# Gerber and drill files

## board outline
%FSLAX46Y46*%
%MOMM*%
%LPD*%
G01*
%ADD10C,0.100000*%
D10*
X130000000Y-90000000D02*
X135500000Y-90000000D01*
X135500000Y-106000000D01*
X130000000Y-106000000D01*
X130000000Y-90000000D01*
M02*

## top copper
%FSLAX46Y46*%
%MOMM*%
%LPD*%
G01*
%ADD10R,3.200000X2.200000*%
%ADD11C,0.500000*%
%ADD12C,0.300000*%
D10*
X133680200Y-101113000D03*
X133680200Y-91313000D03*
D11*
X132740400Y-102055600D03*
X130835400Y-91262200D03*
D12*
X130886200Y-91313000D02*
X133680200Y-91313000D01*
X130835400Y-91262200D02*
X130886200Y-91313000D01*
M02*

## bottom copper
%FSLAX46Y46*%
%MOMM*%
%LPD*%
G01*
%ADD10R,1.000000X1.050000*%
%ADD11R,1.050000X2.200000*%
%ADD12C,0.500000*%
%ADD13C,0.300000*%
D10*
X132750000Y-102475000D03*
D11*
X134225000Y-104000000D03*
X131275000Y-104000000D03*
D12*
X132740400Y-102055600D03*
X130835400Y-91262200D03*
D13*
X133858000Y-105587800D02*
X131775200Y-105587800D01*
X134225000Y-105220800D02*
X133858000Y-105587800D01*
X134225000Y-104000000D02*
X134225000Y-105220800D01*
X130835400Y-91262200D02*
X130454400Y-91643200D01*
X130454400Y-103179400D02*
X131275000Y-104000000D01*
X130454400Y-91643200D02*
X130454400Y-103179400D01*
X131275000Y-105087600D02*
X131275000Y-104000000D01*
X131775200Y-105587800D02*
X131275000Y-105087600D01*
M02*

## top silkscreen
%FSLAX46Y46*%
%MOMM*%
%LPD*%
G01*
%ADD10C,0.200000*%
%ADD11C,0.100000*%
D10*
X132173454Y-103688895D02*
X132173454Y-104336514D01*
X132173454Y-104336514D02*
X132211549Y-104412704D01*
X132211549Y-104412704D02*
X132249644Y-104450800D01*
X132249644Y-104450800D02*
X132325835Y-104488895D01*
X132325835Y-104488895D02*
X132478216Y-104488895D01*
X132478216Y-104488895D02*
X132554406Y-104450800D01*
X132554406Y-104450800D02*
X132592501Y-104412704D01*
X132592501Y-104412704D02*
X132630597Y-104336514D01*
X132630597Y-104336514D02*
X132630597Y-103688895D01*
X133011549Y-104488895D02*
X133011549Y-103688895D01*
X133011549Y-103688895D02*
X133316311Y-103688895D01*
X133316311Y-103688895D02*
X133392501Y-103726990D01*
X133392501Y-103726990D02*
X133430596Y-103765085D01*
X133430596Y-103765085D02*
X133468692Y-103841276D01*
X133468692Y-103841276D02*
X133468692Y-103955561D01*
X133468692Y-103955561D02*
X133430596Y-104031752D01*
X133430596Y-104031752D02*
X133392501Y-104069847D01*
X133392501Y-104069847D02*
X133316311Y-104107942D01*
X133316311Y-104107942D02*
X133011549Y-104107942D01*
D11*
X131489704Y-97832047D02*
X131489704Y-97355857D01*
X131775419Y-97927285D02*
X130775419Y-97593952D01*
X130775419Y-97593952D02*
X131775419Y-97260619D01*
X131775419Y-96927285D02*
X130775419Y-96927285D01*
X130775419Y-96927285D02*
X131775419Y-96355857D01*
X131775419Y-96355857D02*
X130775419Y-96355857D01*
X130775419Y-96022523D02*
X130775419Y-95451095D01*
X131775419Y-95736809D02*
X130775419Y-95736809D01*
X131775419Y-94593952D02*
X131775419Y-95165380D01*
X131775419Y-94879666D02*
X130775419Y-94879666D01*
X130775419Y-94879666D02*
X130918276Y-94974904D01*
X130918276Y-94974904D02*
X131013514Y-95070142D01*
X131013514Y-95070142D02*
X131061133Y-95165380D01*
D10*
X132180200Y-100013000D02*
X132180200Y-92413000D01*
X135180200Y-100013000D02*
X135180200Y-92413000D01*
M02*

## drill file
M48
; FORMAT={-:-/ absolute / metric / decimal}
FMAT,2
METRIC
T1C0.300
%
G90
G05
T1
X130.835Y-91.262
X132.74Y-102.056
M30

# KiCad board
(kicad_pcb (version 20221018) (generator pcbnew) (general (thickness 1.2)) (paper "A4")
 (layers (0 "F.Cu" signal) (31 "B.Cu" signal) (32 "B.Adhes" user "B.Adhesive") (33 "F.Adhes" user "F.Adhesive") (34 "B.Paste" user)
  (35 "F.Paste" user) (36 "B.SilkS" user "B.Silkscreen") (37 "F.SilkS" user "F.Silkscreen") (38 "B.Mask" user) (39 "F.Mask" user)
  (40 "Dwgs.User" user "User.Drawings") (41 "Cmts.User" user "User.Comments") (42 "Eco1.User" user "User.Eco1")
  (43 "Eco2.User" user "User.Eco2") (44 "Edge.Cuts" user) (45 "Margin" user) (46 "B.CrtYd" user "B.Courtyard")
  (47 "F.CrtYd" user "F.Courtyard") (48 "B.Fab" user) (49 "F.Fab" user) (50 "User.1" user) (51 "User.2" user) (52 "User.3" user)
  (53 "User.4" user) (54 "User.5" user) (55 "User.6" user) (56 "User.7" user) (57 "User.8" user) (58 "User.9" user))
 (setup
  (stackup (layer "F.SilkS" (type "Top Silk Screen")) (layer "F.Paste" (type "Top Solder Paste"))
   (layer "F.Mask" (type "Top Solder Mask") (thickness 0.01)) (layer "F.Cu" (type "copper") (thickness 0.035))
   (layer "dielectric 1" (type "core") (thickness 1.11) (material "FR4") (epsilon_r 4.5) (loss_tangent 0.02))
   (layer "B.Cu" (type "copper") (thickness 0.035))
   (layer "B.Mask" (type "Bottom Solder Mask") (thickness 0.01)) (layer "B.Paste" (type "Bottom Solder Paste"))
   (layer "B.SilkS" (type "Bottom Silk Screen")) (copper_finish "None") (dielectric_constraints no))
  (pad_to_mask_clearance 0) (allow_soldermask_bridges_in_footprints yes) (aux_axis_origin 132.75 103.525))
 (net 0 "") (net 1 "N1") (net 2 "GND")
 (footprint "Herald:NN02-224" (layer "F.Cu") (at 133.6802 96.213 90)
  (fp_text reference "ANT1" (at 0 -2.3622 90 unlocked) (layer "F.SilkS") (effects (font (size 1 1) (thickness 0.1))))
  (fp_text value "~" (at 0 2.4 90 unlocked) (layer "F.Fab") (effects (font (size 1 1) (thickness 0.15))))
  (fp_line (start -3.8 -1.5) (end 3.8 -1.5) (stroke (width 0.2) (type default)) (layer "F.SilkS"))
  (fp_line (start -3.8 1.5) (end 3.8 1.5) (stroke (width 0.2) (type default)) (layer "F.SilkS"))
  (pad "1" smd rect (at -4.9 0 90) (size 2.2 3.2) (layers "F.Cu" "F.Paste" "F.Mask") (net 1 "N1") (thermal_bridge_angle 45))
  (pad "2" smd rect (at 4.9 0 90) (size 2.2 3.2) (layers "F.Cu" "F.Paste" "F.Mask") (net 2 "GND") (thermal_bridge_angle 45)))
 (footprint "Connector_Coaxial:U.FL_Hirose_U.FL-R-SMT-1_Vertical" (layer "B.Cu") (at 132.75 103.525 -90)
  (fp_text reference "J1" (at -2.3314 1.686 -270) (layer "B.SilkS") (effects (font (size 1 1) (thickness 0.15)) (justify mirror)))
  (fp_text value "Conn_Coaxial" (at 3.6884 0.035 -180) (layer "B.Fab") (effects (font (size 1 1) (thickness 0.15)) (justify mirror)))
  (pad "1" smd rect (at -1.05 0 270) (size 1.05 1) (layers "B.Cu" "B.Paste" "B.Mask") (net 1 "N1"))
  (pad "2" smd rect (at 0.475 -1.475 270) (size 2.2 1.05) (layers "B.Cu" "B.Paste" "B.Mask") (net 2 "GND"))
  (pad "2" smd rect (at 0.475 1.475 270) (size 2.2 1.05) (layers "B.Cu" "B.Paste" "B.Mask") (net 2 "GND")))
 (gr_rect (start 130 90) (end 135.5 106) (stroke (width 0.1) (type default)) (fill none) (layer "Edge.Cuts"))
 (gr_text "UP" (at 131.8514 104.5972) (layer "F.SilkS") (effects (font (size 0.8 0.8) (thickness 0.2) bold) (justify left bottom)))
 (via (at 132.7404 102.0556) (size 0.5) (drill 0.3) (layers "F.Cu" "B.Cu") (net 1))
 (segment (start 130.8862 91.313) (end 133.6802 91.313) (width 0.3) (layer "F.Cu") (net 2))
 (segment (start 130.8354 91.2622) (end 130.8862 91.313) (width 0.3) (layer "F.Cu") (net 2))
 (via (at 130.8354 91.2622) (size 0.5) (drill 0.3) (layers "F.Cu" "B.Cu") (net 2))
 (segment (start 133.858 105.5878) (end 131.7752 105.5878) (width 0.3) (layer "B.Cu") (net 2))
 (segment (start 134.225 105.2208) (end 133.858 105.5878) (width 0.3) (layer "B.Cu") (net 2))
 (segment (start 134.225 104) (end 134.225 105.2208) (width 0.3) (layer "B.Cu") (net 2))
 (segment (start 130.8354 91.2622) (end 130.4544 91.6432) (width 0.3) (layer "B.Cu") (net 2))
 (segment (start 130.4544 103.1794) (end 131.275 104) (width 0.3) (layer "B.Cu") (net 2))
 (segment (start 130.4544 91.6432) (end 130.4544 103.1794) (width 0.3) (layer "B.Cu") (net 2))
 (segment (start 131.275 105.0876) (end 131.275 104) (width 0.3) (layer "B.Cu") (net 2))
 (segment (start 131.7752 105.5878) (end 131.275 105.0876) (width 0.3) (layer "B.Cu") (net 2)))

